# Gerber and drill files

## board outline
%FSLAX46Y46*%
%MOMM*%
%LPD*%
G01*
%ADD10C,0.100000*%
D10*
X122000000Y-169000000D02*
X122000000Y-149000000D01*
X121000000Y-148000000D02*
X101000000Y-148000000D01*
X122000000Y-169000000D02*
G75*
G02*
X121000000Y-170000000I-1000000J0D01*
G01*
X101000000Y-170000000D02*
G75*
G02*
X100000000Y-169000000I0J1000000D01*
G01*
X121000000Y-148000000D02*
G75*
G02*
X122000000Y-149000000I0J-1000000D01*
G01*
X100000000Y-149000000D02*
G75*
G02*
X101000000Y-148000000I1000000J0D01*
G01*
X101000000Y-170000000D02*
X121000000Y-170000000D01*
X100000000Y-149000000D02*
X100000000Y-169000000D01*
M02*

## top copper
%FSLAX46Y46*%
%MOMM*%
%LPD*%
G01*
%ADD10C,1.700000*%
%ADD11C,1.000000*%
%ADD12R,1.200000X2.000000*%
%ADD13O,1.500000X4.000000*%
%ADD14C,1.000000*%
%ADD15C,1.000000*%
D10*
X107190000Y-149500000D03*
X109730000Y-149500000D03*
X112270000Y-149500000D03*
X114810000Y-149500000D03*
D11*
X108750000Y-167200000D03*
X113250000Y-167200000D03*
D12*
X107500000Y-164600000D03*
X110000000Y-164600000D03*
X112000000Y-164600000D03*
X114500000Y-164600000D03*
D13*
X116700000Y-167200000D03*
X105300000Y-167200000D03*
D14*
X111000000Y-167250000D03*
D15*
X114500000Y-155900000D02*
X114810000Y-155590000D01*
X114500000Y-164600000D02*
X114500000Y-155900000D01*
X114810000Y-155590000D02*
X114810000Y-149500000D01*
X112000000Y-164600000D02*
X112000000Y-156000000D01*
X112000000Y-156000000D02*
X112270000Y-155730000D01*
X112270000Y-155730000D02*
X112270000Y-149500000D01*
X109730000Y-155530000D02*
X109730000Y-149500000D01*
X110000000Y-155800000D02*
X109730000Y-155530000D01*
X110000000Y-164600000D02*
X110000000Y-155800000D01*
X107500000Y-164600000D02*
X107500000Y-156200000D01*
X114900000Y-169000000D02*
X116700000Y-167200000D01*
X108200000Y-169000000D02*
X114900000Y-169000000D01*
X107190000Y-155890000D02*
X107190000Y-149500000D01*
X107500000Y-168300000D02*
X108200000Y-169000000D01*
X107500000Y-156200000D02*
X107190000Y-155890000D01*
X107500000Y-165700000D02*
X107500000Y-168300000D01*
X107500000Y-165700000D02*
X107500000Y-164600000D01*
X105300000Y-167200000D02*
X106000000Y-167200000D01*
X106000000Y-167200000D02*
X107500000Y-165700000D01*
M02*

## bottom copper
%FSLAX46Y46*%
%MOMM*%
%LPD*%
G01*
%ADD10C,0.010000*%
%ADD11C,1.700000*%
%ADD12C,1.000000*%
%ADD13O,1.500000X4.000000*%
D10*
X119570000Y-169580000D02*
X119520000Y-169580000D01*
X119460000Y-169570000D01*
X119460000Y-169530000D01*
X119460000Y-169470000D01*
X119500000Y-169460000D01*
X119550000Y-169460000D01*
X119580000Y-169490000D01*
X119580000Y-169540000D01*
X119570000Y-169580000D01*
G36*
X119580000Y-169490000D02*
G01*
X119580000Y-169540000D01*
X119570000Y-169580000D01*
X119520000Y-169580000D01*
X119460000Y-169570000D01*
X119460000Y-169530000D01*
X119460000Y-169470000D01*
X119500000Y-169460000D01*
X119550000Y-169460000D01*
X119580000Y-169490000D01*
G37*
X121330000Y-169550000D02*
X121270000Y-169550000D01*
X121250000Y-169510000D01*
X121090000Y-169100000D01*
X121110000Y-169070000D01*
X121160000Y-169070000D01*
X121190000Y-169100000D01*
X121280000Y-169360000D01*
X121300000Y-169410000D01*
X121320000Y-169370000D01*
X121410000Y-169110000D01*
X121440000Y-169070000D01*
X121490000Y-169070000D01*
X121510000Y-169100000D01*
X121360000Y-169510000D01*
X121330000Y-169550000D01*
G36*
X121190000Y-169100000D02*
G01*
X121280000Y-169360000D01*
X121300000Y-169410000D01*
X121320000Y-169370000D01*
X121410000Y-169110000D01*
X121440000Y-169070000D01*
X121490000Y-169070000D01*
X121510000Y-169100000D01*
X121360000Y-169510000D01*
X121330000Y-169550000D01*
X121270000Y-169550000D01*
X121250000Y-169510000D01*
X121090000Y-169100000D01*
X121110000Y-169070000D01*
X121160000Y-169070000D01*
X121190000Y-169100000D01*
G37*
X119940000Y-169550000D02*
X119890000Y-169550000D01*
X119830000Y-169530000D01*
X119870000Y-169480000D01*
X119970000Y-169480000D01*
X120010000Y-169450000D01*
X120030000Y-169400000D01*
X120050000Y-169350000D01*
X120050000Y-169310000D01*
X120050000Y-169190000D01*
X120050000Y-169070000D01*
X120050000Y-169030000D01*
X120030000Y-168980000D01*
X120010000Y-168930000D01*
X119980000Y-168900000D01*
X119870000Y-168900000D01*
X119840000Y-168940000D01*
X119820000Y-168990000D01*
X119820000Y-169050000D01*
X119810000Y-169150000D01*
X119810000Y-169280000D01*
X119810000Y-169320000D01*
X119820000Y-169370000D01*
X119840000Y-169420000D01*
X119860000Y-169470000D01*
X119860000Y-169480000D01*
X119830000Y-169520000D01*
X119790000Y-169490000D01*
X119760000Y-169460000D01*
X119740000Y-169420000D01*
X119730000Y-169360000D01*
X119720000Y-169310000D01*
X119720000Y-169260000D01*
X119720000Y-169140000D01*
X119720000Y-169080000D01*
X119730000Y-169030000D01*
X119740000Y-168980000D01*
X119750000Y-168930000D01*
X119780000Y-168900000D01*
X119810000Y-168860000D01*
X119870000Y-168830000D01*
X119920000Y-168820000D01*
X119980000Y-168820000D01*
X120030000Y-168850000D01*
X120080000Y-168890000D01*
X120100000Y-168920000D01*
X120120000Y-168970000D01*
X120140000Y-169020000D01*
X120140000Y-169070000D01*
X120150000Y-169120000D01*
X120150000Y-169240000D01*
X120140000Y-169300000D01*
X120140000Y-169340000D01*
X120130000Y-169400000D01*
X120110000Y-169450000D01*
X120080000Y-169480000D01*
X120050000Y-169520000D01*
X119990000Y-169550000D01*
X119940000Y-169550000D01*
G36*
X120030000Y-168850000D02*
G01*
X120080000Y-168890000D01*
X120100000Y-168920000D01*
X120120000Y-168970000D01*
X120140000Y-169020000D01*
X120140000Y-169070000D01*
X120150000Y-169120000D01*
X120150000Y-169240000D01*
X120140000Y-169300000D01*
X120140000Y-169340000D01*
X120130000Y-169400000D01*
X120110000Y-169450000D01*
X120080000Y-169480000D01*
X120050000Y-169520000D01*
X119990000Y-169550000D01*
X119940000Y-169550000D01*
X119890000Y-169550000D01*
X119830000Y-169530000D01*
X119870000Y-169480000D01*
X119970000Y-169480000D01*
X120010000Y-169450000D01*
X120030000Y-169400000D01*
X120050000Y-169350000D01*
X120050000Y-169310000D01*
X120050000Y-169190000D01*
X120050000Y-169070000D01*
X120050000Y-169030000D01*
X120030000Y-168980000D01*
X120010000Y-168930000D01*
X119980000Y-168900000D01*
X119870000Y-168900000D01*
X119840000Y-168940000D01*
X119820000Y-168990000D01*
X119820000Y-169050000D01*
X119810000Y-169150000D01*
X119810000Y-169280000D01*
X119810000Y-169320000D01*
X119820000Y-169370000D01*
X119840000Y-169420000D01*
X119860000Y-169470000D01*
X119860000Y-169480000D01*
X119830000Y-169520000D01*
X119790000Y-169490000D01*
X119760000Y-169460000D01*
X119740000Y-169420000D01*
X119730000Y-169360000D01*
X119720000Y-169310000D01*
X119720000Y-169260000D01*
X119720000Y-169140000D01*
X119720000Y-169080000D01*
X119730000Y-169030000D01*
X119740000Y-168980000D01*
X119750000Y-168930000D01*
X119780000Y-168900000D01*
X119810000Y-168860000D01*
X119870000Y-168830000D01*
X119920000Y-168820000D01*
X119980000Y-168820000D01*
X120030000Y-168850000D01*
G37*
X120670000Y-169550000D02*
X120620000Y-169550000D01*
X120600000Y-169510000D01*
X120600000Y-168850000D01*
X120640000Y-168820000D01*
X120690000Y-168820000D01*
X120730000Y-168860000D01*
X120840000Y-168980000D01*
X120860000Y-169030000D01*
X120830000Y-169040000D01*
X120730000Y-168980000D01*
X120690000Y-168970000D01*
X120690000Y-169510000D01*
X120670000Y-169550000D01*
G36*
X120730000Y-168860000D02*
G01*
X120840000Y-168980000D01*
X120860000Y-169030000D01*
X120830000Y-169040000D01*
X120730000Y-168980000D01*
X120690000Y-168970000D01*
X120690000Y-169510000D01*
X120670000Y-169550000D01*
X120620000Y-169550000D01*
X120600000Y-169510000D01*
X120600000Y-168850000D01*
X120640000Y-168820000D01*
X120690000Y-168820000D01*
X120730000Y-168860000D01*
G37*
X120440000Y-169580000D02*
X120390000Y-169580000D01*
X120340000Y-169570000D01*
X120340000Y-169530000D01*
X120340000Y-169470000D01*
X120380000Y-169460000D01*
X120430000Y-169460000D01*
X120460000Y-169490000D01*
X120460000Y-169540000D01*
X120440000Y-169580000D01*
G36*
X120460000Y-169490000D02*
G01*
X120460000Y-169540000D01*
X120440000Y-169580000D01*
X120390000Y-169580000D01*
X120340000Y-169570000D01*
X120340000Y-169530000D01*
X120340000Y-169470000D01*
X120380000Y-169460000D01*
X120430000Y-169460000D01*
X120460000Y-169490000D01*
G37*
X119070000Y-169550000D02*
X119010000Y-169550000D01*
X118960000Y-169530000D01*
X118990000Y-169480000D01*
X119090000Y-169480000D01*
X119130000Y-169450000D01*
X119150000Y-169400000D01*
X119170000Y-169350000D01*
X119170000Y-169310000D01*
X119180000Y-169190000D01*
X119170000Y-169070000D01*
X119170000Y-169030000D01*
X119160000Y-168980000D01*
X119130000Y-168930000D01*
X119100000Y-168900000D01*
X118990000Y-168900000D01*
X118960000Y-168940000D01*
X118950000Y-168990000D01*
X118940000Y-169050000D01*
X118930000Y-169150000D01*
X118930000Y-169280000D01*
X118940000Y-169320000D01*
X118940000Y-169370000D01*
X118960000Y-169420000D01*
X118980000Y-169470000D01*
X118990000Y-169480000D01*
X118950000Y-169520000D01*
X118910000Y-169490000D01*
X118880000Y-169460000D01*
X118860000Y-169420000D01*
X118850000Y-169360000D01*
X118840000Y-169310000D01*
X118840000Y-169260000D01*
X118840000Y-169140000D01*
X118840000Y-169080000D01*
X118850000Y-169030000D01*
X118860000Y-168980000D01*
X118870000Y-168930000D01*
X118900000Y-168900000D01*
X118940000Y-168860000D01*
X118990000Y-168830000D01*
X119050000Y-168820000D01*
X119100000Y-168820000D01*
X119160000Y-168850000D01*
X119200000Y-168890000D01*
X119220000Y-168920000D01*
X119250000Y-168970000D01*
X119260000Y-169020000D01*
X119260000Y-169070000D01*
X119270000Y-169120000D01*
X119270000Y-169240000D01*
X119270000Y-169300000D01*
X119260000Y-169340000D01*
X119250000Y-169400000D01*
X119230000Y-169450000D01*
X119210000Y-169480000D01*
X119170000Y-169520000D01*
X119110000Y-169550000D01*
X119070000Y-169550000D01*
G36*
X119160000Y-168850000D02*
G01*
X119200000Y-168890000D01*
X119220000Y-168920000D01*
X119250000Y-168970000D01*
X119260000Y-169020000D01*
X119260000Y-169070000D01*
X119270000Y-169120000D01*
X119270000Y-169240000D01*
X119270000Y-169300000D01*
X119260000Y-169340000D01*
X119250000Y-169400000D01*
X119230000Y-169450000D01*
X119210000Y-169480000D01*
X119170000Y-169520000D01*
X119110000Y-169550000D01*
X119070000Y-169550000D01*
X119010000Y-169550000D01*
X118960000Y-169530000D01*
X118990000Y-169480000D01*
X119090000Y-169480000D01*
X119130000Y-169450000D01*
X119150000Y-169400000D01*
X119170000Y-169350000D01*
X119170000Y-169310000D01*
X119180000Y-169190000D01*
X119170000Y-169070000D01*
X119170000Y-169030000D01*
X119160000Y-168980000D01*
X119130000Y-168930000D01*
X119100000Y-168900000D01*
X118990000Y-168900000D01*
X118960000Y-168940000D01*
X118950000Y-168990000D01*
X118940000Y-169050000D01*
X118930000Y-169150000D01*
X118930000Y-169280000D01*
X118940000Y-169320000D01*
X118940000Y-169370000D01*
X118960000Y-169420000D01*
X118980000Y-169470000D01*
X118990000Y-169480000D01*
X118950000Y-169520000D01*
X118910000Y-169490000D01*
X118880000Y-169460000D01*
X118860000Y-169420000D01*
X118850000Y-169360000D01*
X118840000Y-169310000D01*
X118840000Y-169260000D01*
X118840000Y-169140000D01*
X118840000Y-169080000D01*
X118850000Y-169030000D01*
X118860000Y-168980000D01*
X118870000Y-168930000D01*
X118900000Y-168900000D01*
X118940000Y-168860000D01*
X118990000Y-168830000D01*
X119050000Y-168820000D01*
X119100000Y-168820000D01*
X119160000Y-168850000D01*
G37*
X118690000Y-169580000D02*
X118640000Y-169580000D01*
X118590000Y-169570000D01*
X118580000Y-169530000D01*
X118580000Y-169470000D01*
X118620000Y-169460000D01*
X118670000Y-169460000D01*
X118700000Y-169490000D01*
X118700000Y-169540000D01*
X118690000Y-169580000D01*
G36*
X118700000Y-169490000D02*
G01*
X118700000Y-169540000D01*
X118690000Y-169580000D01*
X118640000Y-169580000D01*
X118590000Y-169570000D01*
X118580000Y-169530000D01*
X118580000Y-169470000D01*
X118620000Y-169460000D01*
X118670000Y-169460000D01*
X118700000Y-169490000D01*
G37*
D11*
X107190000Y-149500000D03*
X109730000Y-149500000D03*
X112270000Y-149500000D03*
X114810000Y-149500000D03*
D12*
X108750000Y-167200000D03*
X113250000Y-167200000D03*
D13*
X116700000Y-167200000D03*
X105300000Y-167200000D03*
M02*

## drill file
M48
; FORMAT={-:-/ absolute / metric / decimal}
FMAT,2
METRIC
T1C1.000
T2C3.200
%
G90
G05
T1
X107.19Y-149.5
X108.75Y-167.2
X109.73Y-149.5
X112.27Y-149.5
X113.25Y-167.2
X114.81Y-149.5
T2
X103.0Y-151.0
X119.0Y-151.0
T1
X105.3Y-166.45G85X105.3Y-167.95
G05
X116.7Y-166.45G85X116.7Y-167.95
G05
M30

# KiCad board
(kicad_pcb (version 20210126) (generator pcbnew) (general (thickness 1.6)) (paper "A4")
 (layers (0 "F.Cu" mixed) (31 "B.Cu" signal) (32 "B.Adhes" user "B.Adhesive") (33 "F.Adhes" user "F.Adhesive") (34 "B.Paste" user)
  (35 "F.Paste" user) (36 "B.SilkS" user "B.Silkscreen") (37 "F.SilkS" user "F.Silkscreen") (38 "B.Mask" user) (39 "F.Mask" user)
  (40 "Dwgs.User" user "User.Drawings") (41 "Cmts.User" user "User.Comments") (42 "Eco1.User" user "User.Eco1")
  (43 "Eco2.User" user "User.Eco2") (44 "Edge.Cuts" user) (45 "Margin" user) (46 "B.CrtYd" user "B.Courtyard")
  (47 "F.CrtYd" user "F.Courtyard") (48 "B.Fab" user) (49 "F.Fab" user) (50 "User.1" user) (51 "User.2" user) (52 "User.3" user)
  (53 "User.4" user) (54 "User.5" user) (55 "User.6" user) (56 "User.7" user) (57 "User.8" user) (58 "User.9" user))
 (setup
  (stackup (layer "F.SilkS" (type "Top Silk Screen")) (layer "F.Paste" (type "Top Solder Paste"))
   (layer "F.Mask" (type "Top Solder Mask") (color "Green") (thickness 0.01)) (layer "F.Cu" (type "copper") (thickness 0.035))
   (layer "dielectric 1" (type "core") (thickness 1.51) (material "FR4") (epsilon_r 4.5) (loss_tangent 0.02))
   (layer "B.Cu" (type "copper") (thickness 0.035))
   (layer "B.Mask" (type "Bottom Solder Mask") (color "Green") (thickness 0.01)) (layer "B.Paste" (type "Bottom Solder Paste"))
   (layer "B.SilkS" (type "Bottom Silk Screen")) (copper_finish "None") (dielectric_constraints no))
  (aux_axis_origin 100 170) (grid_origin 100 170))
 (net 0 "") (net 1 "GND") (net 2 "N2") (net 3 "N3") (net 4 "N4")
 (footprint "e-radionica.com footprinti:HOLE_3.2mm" (layer "F.Cu") (at 103 151)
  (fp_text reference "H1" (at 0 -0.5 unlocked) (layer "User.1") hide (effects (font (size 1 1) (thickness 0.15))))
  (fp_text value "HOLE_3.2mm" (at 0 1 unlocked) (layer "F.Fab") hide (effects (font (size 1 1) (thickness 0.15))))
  (pad "" np_thru_hole circle (at 0 0) (locked) (size 3.2 3.2) (drill 3.2) (layers F&B.Cu *.Mask)))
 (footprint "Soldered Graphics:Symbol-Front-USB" (layer "F.Cu") (at 120 166)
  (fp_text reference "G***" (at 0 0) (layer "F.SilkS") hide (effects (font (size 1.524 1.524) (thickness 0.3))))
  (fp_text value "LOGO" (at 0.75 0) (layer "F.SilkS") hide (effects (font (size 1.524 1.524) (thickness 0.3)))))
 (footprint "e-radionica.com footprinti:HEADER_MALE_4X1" (layer "F.Cu") (at 111 149.5)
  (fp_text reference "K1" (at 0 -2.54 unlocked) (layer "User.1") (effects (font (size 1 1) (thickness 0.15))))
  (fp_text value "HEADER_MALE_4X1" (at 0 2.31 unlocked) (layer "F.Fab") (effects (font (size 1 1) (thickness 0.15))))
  (pad "1" thru_hole circle (at -3.81 0) (locked) (size 1.7 1.7) (drill 1) (layers *.Cu *.Mask) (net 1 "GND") (solder_mask_margin 0.1))
  (pad "2" thru_hole circle (at -1.27 0) (locked) (size 1.7 1.7) (drill 1) (layers *.Cu *.Mask) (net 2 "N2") (solder_mask_margin 0.1))
  (pad "3" thru_hole circle (at 1.27 0) (locked) (size 1.7 1.7) (drill 1) (layers *.Cu *.Mask) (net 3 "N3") (solder_mask_margin 0.1))
  (pad "4" thru_hole circle (at 3.81 0) (locked) (size 1.7 1.7) (drill 1) (layers *.Cu *.Mask) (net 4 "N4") (solder_mask_margin 0.1)))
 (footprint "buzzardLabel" (layer "F.Cu") (at 111 161.5)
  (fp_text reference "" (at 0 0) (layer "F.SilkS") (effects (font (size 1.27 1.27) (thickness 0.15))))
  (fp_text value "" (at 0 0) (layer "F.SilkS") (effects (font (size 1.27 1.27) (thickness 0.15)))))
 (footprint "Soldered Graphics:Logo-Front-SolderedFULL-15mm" (layer "F.Cu") (at 111 157)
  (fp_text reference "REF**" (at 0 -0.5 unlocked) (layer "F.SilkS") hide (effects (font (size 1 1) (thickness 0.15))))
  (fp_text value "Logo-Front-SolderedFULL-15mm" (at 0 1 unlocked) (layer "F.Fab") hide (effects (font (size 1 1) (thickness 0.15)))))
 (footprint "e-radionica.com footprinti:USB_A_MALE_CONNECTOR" (layer "F.Cu") (at 111 164.6)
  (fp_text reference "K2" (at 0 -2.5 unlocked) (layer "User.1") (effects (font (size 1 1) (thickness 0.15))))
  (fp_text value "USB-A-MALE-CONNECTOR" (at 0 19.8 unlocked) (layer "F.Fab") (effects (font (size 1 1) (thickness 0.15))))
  (pad "" thru_hole circle (at -2.25 2.6) (locked) (size 1 1) (drill 1) (layers *.Cu *.Mask) (solder_mask_margin 0.1))
  (pad "" thru_hole circle (at 2.25 2.6) (locked) (size 1 1) (drill 1) (layers *.Cu *.Mask) (solder_mask_margin 0.1))
  (pad "1" smd rect (at -3.5 0) (locked) (size 1.2 2) (layers "F.Cu" "F.Paste" "F.Mask") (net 1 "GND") (solder_mask_margin 0.1))
  (pad "2" smd rect (at -1 0) (locked) (size 1.2 2) (layers "F.Cu" "F.Paste" "F.Mask") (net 2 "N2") (solder_mask_margin 0.1))
  (pad "3" smd rect (at 1 0) (locked) (size 1.2 2) (layers "F.Cu" "F.Paste" "F.Mask") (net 3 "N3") (solder_mask_margin 0.1))
  (pad "4" smd rect (at 3.5 0) (locked) (size 1.2 2) (layers "F.Cu" "F.Paste" "F.Mask") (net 4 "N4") (solder_mask_margin 0.1))
  (pad "5" thru_hole oval (at 5.7 2.6) (locked) (size 1.5 4) (drill oval 1 2.5) (layers *.Cu *.Mask) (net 1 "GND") (solder_mask_margin 0.1))
  (pad "5" thru_hole oval (at -5.7 2.6) (locked) (size 1.5 4) (drill oval 1 2.5) (layers *.Cu *.Mask) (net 1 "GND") (solder_mask_margin 0.1)))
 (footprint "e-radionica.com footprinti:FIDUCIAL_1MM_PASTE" (layer "F.Cu") (at 111 167.25)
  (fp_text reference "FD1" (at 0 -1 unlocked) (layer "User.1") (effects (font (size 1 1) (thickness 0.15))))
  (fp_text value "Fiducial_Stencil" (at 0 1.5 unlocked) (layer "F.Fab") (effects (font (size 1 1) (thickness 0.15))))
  (pad "1" smd circle (at 0 0) (locked) (size 1 1) (layers "F.Cu" "F.Paste" "F.Mask")))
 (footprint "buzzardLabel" (layer "F.Cu") (at 107.19 147.6 90)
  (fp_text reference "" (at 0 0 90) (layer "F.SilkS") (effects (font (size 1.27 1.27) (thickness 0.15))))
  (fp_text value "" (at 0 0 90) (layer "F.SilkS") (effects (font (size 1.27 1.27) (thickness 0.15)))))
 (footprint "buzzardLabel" (layer "F.Cu") (at 114.81 147.6 90)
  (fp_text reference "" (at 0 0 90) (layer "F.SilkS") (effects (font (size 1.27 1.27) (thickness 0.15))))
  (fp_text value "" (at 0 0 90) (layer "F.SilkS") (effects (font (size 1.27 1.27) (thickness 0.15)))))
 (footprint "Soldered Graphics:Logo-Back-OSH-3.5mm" (layer "F.Cu") (at 111 164)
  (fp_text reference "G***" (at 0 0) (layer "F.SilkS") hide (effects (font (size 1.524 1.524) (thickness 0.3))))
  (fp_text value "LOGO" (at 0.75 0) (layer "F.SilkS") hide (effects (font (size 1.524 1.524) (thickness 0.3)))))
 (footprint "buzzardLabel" (layer "F.Cu") (at 112.27 147.6 90)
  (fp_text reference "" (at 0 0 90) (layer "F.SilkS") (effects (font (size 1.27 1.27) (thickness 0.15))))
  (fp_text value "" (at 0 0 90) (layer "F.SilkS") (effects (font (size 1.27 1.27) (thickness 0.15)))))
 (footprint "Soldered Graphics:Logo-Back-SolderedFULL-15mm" (layer "F.Cu") (at 111 157)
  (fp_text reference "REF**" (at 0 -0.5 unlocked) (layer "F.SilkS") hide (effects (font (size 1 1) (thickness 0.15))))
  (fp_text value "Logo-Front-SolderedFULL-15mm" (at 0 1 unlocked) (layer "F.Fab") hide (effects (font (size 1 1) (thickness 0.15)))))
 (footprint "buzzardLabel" (layer "F.Cu") (at 109.73 147.6 90)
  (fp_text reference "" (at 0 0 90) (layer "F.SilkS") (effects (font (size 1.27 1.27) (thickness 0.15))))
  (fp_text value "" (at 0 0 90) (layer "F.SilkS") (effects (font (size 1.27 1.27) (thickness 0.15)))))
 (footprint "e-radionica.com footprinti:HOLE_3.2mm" (layer "F.Cu") (at 119 151)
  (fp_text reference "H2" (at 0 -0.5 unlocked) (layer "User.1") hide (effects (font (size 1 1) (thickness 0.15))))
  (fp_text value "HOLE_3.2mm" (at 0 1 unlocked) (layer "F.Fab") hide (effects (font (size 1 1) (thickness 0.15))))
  (pad "" np_thru_hole circle (at 0 0) (locked) (size 3.2 3.2) (drill 3.2) (layers F&B.Cu *.Mask)))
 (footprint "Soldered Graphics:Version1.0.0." (layer "B.Cu") (at 120 169.2 180)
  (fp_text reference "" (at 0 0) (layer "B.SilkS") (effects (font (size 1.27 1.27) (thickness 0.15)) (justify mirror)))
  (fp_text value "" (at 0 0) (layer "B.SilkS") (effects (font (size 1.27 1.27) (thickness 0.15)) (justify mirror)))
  (fp_poly
   (pts (xy 0.43 -0.38) (xy 0.48 -0.38) (xy 0.54 -0.37) (xy 0.54 -0.33) (xy 0.54 -0.27) (xy 0.5 -0.26) (xy 0.45 -0.26) (xy 0.42 -0.29)
    (xy 0.42 -0.34) (xy 0.43 -0.38))
   (layer "B.Cu") (width 0.01) (fill solid))
  (fp_poly
   (pts (xy -1.33 -0.35) (xy -1.27 -0.35) (xy -1.25 -0.31) (xy -1.09 0.1) (xy -1.11 0.13) (xy -1.16 0.13) (xy -1.19 0.1) (xy -1.28 -0.16)
    (xy -1.3 -0.21) (xy -1.32 -0.17) (xy -1.41 0.09) (xy -1.44 0.13) (xy -1.49 0.13) (xy -1.51 0.1) (xy -1.36 -0.31) (xy -1.33 -0.35))
   (layer "B.Cu") (width 0.01) (fill solid))
  (fp_poly
   (pts (xy 0.06 -0.35) (xy 0.11 -0.35) (xy 0.17 -0.33) (xy 0.13 -0.28) (xy 0.03 -0.28) (xy -0.01 -0.25) (xy -0.03 -0.2) (xy -0.05 -0.15)
    (xy -0.05 -0.11) (xy -0.05 0.01) (xy -0.05 0.13) (xy -0.05 0.17) (xy -0.03 0.22) (xy -0.01 0.27) (xy 0.02 0.3) (xy 0.13 0.3)
    (xy 0.16 0.26) (xy 0.18 0.21) (xy 0.18 0.15) (xy 0.19 0.05) (xy 0.19 -0.08) (xy 0.19 -0.12) (xy 0.18 -0.17) (xy 0.16 -0.22)
    (xy 0.14 -0.27) (xy 0.14 -0.28) (xy 0.17 -0.32) (xy 0.21 -0.29) (xy 0.24 -0.26) (xy 0.26 -0.22) (xy 0.27 -0.16) (xy 0.28 -0.11)
    (xy 0.28 -0.06) (xy 0.28 0.06) (xy 0.28 0.12) (xy 0.27 0.17) (xy 0.26 0.22) (xy 0.25 0.27) (xy 0.22 0.3) (xy 0.19 0.34) (xy 0.13 0.37)
    (xy 0.08 0.38) (xy 0.02 0.38) (xy -0.03 0.35) (xy -0.08 0.31) (xy -0.1 0.28) (xy -0.12 0.23) (xy -0.14 0.18) (xy -0.14 0.13)
    (xy -0.15 0.08) (xy -0.15 -0.04) (xy -0.14 -0.1) (xy -0.14 -0.14) (xy -0.13 -0.2) (xy -0.11 -0.25) (xy -0.08 -0.28) (xy -0.05 -0.32)
    (xy 0.01 -0.35) (xy 0.06 -0.35))
   (layer "B.Cu") (width 0.01) (fill solid))
  (fp_poly
   (pts (xy -0.67 -0.35) (xy -0.62 -0.35) (xy -0.6 -0.31) (xy -0.6 0.35) (xy -0.64 0.38) (xy -0.69 0.38) (xy -0.73 0.34) (xy -0.84 0.22)
    (xy -0.86 0.17) (xy -0.83 0.16) (xy -0.73 0.22) (xy -0.69 0.23) (xy -0.69 -0.31) (xy -0.67 -0.35))
   (layer "B.Cu") (width 0.01) (fill solid))
  (fp_poly
   (pts (xy -0.44 -0.38) (xy -0.39 -0.38) (xy -0.34 -0.37) (xy -0.34 -0.33) (xy -0.34 -0.27) (xy -0.38 -0.26) (xy -0.43 -0.26)
    (xy -0.46 -0.29) (xy -0.46 -0.34) (xy -0.44 -0.38))
   (layer "B.Cu") (width 0.01) (fill solid))
  (fp_poly
   (pts (xy 0.93 -0.35) (xy 0.99 -0.35) (xy 1.04 -0.33) (xy 1.01 -0.28) (xy 0.91 -0.28) (xy 0.87 -0.25) (xy 0.85 -0.2) (xy 0.83 -0.15)
    (xy 0.83 -0.11) (xy 0.82 0.01) (xy 0.83 0.13) (xy 0.83 0.17) (xy 0.84 0.22) (xy 0.87 0.27) (xy 0.9 0.3) (xy 1.01 0.3) (xy 1.04 0.26)
    (xy 1.05 0.21) (xy 1.06 0.15) (xy 1.07 0.05) (xy 1.07 -0.08) (xy 1.06 -0.12) (xy 1.06 -0.17) (xy 1.04 -0.22) (xy 1.02 -0.27)
    (xy 1.01 -0.28) (xy 1.05 -0.32) (xy 1.09 -0.29) (xy 1.12 -0.26) (xy 1.14 -0.22) (xy 1.15 -0.16) (xy 1.16 -0.11) (xy 1.16 -0.06)
    (xy 1.16 0.06) (xy 1.16 0.12) (xy 1.15 0.17) (xy 1.14 0.22) (xy 1.13 0.27) (xy 1.1 0.3) (xy 1.06 0.34) (xy 1.01 0.37) (xy 0.95 0.38)
    (xy 0.9 0.38) (xy 0.84 0.35) (xy 0.8 0.31) (xy 0.78 0.28) (xy 0.75 0.23) (xy 0.74 0.18) (xy 0.74 0.13) (xy 0.73 0.08) (xy 0.73 -0.04)
    (xy 0.73 -0.1) (xy 0.74 -0.14) (xy 0.75 -0.2) (xy 0.77 -0.25) (xy 0.79 -0.28) (xy 0.83 -0.32) (xy 0.89 -0.35) (xy 0.93 -0.35))
   (layer "B.Cu") (width 0.01) (fill solid))
  (fp_poly
   (pts (xy 1.31 -0.38) (xy 1.36 -0.38) (xy 1.41 -0.37) (xy 1.42 -0.33) (xy 1.42 -0.27) (xy 1.38 -0.26) (xy 1.33 -0.26) (xy 1.3 -0.29)
    (xy 1.3 -0.34) (xy 1.31 -0.38))
   (layer "B.Cu") (width 0.01) (fill solid)))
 (gr_line (start 122 169) (end 122 149) (layer "Edge.Cuts") (width 0.1))
 (gr_line (start 121 148) (end 101 148) (layer "Edge.Cuts") (width 0.1))
 (gr_arc (start 121 169) (end 121 170) (angle -90) (layer "Edge.Cuts") (width 0.1))
 (gr_arc (start 101 169) (end 101 170) (angle 90) (layer "Edge.Cuts") (width 0.1))
 (gr_arc (start 121 149) (end 121 148) (angle 90) (layer "Edge.Cuts") (width 0.1))
 (gr_arc (start 101 149) (end 101 148) (angle -90) (layer "Edge.Cuts") (width 0.1))
 (gr_line (start 101 170) (end 121 170) (layer "Edge.Cuts") (width 0.1))
 (gr_line (start 100 149) (end 100 169) (layer "Edge.Cuts") (width 0.1))
 (segment (start 114.5 155.9) (end 114.81 155.59) (width 1) (layer "F.Cu") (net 4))
 (segment (start 114.5 164.6) (end 114.5 155.9) (width 1) (layer "F.Cu") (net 4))
 (segment (start 114.81 155.59) (end 114.81 149.5) (width 1) (layer "F.Cu") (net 4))
 (segment (start 112 164.6) (end 112 156) (width 1) (layer "F.Cu") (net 3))
 (segment (start 112 156) (end 112.27 155.73) (width 1) (layer "F.Cu") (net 3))
 (segment (start 112.27 155.73) (end 112.27 149.5) (width 1) (layer "F.Cu") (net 3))
 (segment (start 109.73 155.53) (end 109.73 149.5) (width 1) (layer "F.Cu") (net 2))
 (segment (start 110 155.8) (end 109.73 155.53) (width 1) (layer "F.Cu") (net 2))
 (segment (start 110 164.6) (end 110 155.8) (width 1) (layer "F.Cu") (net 2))
 (segment (start 107.5 164.6) (end 107.5 156.2) (width 1) (layer "F.Cu") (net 1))
 (segment (start 114.9 169) (end 116.7 167.2) (width 1) (layer "F.Cu") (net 1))
 (segment (start 108.2 169) (end 114.9 169) (width 1) (layer "F.Cu") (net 1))
 (segment (start 107.19 155.89) (end 107.19 149.5) (width 1) (layer "F.Cu") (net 1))
 (segment (start 107.5 168.3) (end 108.2 169) (width 1) (layer "F.Cu") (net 1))
 (segment (start 107.5 156.2) (end 107.19 155.89) (width 1) (layer "F.Cu") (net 1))
 (segment (start 107.5 165.7) (end 107.5 168.3) (width 1) (layer "F.Cu") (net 1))
 (segment (start 107.5 165.7) (end 107.5 164.6) (width 1) (layer "F.Cu") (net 1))
 (segment (start 105.3 167.2) (end 106 167.2) (width 1) (layer "F.Cu") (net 1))
 (segment (start 106 167.2) (end 107.5 165.7) (width 1) (layer "F.Cu") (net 1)))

